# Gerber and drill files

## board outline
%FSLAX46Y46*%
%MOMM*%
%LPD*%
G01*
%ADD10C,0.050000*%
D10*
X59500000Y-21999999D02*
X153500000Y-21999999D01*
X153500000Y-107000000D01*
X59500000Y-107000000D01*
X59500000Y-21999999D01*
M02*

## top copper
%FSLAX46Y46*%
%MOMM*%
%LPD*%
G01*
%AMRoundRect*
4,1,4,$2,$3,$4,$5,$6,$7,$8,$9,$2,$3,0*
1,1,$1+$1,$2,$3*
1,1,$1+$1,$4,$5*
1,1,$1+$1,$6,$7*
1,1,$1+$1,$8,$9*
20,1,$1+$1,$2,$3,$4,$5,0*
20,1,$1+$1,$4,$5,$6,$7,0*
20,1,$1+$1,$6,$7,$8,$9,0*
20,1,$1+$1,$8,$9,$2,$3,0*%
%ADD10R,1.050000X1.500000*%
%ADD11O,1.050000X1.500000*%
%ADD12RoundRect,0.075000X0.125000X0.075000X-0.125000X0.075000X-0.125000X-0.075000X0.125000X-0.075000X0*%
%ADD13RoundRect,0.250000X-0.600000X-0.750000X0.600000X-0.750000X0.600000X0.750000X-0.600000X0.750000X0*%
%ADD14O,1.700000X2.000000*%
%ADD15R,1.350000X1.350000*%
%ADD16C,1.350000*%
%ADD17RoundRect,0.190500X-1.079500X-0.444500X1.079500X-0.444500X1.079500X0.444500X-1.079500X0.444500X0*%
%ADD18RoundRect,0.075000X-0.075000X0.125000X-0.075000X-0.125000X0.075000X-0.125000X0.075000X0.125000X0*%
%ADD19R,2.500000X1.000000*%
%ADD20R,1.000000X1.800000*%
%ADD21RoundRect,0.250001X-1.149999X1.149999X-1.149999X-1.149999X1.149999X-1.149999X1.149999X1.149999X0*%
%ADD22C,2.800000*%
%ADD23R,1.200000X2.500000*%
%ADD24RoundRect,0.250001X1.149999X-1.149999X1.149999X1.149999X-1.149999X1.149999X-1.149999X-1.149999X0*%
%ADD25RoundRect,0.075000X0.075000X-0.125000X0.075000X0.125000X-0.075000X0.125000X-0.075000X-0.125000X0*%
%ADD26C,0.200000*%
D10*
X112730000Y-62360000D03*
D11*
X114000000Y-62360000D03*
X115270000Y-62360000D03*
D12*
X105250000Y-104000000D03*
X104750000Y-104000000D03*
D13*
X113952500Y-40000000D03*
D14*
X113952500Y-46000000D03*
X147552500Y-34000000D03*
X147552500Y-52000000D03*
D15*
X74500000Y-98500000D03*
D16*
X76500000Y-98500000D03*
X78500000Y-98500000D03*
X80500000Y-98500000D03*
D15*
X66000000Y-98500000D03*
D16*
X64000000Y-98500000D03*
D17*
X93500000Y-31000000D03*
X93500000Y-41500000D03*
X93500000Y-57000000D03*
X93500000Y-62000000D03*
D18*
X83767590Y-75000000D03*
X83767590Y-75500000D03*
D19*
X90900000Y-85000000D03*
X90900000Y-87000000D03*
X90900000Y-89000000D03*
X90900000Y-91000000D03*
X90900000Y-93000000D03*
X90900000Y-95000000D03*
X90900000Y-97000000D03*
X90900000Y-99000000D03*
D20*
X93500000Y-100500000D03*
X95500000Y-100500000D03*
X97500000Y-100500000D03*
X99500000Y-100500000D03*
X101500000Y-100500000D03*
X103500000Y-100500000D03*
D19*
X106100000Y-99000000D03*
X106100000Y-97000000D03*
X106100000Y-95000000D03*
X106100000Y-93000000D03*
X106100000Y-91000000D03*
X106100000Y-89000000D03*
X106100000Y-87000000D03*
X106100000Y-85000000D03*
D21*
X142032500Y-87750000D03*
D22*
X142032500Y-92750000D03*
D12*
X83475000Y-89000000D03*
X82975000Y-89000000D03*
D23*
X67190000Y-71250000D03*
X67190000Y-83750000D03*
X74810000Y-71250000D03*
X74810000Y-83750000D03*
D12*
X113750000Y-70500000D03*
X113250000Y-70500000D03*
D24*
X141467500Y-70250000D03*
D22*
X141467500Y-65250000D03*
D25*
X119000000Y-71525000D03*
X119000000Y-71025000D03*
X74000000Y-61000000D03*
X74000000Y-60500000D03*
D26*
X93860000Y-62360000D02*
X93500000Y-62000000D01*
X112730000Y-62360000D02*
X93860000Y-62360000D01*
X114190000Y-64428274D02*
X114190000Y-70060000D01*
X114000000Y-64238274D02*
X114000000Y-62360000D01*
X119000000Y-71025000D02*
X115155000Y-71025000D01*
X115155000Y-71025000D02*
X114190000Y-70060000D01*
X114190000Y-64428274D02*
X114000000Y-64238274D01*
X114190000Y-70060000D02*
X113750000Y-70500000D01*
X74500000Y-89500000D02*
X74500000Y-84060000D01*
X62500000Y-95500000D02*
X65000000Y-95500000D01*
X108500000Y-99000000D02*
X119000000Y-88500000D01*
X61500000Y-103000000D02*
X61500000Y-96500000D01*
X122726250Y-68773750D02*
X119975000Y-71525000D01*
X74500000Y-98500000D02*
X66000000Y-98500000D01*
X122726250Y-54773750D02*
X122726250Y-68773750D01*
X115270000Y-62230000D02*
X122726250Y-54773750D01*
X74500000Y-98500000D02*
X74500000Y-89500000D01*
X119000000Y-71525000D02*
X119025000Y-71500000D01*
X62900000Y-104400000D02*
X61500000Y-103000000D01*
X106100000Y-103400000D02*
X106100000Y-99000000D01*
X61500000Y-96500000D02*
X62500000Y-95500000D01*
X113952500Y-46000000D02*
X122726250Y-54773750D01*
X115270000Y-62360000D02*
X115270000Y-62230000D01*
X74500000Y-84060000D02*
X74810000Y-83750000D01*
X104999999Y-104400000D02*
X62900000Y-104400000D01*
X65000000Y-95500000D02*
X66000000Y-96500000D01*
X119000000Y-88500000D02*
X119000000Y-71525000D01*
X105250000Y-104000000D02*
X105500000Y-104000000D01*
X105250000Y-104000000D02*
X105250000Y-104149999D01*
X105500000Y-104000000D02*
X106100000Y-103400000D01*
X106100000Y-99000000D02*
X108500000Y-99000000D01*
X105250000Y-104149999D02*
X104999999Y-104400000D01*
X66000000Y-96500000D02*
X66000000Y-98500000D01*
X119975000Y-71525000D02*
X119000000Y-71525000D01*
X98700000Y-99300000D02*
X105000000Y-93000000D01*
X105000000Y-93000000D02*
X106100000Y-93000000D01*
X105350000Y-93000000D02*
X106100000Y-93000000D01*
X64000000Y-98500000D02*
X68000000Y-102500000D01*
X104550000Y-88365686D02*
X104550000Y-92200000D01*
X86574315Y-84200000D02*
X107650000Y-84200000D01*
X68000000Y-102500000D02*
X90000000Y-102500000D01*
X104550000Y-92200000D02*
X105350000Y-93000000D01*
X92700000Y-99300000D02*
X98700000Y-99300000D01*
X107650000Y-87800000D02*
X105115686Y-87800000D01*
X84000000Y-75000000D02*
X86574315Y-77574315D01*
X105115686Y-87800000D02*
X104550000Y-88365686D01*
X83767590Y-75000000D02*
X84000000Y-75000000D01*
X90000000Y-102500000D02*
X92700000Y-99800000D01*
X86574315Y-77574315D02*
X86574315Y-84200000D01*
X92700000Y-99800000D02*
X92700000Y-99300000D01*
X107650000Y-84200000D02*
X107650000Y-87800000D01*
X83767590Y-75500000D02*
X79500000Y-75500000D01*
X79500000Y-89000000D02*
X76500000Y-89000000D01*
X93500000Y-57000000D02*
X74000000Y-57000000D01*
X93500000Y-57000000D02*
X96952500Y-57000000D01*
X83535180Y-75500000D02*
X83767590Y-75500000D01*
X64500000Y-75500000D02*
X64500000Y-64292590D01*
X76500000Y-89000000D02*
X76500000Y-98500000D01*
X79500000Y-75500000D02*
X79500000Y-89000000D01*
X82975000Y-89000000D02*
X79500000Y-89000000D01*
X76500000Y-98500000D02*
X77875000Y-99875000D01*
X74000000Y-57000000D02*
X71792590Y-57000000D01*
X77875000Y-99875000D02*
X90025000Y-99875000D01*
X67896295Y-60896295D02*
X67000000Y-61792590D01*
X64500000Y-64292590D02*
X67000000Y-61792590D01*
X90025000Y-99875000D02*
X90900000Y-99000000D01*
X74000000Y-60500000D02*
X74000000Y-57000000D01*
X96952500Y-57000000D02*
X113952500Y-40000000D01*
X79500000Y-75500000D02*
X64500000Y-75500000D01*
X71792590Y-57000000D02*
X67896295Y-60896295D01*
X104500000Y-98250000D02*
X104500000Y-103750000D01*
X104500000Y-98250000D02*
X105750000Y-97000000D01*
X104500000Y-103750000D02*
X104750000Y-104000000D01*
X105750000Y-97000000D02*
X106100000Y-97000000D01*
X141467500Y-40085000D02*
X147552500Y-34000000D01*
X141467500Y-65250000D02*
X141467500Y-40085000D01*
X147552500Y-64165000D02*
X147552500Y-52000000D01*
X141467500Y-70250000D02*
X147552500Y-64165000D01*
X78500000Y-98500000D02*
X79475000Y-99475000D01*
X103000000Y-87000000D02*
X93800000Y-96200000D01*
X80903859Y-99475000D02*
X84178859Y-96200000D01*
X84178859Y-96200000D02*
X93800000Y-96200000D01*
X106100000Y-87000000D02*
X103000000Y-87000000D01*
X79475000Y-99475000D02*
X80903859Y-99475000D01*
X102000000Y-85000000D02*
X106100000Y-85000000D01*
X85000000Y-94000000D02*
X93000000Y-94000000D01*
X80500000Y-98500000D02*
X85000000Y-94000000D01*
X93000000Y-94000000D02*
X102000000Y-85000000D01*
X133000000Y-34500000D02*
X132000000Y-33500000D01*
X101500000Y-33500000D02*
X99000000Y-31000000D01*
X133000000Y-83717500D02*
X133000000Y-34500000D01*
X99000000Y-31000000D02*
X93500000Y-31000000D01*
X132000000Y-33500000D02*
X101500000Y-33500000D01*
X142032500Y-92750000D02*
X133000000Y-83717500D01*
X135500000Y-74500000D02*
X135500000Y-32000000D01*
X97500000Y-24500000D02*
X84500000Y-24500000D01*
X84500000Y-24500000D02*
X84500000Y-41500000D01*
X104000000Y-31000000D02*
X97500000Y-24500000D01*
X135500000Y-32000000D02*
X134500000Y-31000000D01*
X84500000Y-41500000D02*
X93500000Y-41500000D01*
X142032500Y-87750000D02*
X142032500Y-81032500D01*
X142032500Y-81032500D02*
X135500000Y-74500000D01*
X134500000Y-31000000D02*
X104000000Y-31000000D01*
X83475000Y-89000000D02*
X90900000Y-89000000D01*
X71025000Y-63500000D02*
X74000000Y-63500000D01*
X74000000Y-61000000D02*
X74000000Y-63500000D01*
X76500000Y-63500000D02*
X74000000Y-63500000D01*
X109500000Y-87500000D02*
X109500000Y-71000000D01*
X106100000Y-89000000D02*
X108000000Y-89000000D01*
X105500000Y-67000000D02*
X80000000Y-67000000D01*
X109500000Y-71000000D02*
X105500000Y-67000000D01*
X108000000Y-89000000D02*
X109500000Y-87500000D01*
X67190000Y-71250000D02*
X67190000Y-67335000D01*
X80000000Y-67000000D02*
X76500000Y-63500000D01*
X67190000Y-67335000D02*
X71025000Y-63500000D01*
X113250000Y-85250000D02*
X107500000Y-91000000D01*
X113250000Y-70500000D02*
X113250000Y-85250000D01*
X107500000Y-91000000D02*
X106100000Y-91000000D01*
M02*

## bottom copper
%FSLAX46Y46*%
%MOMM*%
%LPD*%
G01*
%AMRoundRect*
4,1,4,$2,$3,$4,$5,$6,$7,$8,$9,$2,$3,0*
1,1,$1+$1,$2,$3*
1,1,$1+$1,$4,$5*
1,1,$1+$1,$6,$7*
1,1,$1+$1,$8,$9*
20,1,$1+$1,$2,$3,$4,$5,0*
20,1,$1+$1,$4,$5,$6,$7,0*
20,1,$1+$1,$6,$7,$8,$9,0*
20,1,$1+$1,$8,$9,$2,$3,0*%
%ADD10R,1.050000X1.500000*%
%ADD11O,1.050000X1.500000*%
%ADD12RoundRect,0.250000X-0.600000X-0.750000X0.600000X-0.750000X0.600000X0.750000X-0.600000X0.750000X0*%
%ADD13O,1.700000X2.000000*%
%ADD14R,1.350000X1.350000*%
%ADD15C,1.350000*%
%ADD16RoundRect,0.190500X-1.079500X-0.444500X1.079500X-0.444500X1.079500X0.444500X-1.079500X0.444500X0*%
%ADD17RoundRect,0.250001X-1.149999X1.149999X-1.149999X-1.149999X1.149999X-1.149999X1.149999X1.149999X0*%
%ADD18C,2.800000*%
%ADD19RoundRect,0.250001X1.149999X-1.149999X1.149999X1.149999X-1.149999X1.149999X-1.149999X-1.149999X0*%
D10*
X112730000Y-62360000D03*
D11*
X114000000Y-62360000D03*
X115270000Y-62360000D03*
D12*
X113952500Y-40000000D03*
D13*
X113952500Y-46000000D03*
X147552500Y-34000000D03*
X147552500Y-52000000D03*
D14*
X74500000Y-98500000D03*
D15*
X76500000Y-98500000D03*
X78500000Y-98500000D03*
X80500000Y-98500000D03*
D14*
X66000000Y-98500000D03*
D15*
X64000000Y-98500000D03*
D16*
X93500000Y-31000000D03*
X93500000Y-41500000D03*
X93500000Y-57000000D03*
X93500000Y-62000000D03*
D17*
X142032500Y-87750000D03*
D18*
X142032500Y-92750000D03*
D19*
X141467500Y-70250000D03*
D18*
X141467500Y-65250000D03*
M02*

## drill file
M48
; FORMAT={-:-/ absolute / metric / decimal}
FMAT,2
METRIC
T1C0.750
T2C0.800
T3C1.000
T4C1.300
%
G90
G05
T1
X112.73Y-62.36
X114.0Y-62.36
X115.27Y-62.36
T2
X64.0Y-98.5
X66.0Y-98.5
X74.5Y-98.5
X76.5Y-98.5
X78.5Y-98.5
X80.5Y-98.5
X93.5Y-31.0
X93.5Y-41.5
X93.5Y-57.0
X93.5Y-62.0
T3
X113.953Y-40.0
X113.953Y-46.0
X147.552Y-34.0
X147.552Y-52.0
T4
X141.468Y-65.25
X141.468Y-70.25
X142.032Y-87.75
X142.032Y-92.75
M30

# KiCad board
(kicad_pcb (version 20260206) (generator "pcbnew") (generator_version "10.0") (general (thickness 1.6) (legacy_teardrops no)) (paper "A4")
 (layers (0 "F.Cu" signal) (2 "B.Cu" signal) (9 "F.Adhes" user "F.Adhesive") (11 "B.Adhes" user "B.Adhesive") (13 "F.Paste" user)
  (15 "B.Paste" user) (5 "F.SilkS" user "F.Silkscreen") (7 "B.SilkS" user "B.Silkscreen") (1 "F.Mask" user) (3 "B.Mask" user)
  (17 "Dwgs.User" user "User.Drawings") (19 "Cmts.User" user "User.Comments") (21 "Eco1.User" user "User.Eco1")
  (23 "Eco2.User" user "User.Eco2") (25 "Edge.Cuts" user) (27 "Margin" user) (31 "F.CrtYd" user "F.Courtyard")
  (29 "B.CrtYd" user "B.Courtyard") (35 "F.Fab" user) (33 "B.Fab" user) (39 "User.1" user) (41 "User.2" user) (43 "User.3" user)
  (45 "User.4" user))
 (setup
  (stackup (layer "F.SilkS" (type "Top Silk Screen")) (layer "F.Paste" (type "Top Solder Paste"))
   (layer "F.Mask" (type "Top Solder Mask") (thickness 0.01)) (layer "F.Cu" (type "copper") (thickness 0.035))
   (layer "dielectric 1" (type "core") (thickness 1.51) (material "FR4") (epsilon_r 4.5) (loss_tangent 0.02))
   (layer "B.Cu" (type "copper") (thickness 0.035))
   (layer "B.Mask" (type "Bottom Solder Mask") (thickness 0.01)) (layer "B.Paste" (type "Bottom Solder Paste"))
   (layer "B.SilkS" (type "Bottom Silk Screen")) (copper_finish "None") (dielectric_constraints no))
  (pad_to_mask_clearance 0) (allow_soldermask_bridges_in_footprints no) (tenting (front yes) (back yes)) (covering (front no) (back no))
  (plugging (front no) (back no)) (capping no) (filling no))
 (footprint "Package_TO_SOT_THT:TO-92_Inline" (layer "F.Cu") (at 112.73 62.36)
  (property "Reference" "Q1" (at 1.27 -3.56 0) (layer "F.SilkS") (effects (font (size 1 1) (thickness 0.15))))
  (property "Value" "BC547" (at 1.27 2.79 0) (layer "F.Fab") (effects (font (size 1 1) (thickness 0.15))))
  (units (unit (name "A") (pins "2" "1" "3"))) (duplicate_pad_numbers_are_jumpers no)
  (pad "1" thru_hole rect (at 0 0) (size 1.05 1.5) (drill 0.75) (layers "*.Cu" "*.Mask") (remove_unused_layers no) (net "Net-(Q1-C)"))
  (pad "2" thru_hole oval (at 1.27 0) (size 1.05 1.5) (drill 0.75) (layers "*.Cu" "*.Mask") (remove_unused_layers no) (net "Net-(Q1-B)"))
  (pad "3" thru_hole oval (at 2.54 0) (size 1.05 1.5) (drill 0.75) (layers "*.Cu" "*.Mask") (remove_unused_layers no) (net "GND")))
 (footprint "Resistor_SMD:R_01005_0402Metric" (layer "F.Cu") (at 105 104 180)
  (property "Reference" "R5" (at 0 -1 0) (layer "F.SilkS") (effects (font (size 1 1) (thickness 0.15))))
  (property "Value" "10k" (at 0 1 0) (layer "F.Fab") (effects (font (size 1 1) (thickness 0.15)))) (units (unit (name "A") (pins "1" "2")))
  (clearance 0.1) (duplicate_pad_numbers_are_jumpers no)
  (pad "" smd roundrect (at -0.275 0 180) (size 0.27 0.27) (layers "F.Paste") (roundrect_rratio 0.25))
  (pad "" smd roundrect (at 0.275 0 180) (size 0.27 0.27) (layers "F.Paste") (roundrect_rratio 0.25))
  (pad "1" smd roundrect (at -0.25 0 180) (size 0.4 0.3) (layers "F.Cu" "F.Mask") (roundrect_rratio 0.25) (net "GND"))
  (pad "2" smd roundrect (at 0.25 0 180) (size 0.4 0.3) (layers "F.Cu" "F.Mask") (roundrect_rratio 0.25) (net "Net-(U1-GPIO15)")))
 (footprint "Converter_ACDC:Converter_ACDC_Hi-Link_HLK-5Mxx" (layer "F.Cu") (at 113.9525 40)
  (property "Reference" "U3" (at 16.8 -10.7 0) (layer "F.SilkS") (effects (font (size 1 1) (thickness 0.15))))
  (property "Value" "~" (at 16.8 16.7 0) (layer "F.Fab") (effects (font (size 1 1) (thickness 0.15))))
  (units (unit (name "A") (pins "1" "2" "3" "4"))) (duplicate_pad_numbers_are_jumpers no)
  (pad "1" thru_hole roundrect (at 0 0) (size 1.7 2) (drill 1) (layers "*.Cu" "*.Mask") (remove_unused_layers no)
   (roundrect_rratio 0.147059) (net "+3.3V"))
  (pad "2" thru_hole oval (at 0 6) (size 1.7 2) (drill 1) (layers "*.Cu" "*.Mask") (remove_unused_layers no) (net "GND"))
  (pad "3" thru_hole oval (at 33.6 -6) (size 1.7 2) (drill 1) (layers "*.Cu" "*.Mask") (remove_unused_layers no) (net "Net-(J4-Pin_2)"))
  (pad "4" thru_hole oval (at 33.6 12) (size 1.7 2) (drill 1) (layers "*.Cu" "*.Mask") (remove_unused_layers no) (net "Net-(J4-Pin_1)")))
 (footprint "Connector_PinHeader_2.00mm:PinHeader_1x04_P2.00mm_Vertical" (layer "F.Cu") (at 74.5 98.5 90)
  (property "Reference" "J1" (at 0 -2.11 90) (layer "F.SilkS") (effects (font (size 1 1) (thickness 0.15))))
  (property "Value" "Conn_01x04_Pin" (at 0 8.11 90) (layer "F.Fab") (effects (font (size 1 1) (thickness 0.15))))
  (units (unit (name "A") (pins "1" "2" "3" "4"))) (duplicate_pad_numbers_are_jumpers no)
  (pad "1" thru_hole rect (at 0 0 90) (size 1.35 1.35) (drill 0.8) (layers "*.Cu" "*.Mask") (remove_unused_layers no) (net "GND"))
  (pad "2" thru_hole circle (at 0 2 90) (size 1.35 1.35) (drill 0.8) (layers "*.Cu" "*.Mask") (remove_unused_layers no) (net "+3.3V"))
  (pad "3" thru_hole circle (at 0 4 90) (size 1.35 1.35) (drill 0.8) (layers "*.Cu" "*.Mask") (remove_unused_layers no)
   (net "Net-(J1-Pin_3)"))
  (pad "4" thru_hole circle (at 0 6 90) (size 1.35 1.35) (drill 0.8) (layers "*.Cu" "*.Mask") (remove_unused_layers no)
   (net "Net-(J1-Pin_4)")))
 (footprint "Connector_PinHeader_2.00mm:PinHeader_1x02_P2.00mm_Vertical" (layer "F.Cu") (at 66 98.5 -90)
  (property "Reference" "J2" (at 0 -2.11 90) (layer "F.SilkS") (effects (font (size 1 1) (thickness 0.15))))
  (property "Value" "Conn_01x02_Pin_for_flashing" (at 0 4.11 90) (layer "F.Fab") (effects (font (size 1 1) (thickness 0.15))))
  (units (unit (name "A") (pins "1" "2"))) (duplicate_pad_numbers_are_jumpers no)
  (pad "1" thru_hole rect (at 0 0 270) (size 1.35 1.35) (drill 0.8) (layers "*.Cu" "*.Mask") (remove_unused_layers no) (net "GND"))
  (pad "2" thru_hole circle (at 0 2 270) (size 1.35 1.35) (drill 0.8) (layers "*.Cu" "*.Mask") (remove_unused_layers no)
   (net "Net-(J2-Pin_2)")))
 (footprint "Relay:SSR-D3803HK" (layer "F.Cu") (at 93.5 46.5)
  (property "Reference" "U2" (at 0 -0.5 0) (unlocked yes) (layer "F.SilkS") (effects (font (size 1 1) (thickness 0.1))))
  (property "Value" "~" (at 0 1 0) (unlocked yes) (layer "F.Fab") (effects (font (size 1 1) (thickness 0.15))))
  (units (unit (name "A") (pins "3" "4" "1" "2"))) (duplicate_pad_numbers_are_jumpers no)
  (pad "1" thru_hole roundrect (at 0 -15.5) (size 2.54 1.27) (drill 0.8) (layers "*.Cu" "*.Mask") (remove_unused_layers no)
   (roundrect_rratio 0.15) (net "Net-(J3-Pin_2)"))
  (pad "2" thru_hole roundrect (at 0 -5) (size 2.54 1.27) (drill 0.8) (layers "*.Cu" "*.Mask") (remove_unused_layers no)
   (roundrect_rratio 0.15) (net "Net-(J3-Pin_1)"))
  (pad "3" thru_hole roundrect (at 0 10.5) (size 2.54 1.27) (drill 0.8) (layers "*.Cu" "*.Mask") (remove_unused_layers no)
   (roundrect_rratio 0.15) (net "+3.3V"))
  (pad "4" thru_hole roundrect (at 0 15.5) (size 2.54 1.27) (drill 0.8) (layers "*.Cu" "*.Mask") (remove_unused_layers no)
   (roundrect_rratio 0.15) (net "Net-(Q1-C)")))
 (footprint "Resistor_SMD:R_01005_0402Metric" (layer "F.Cu") (at 83.76759 75.25 -90)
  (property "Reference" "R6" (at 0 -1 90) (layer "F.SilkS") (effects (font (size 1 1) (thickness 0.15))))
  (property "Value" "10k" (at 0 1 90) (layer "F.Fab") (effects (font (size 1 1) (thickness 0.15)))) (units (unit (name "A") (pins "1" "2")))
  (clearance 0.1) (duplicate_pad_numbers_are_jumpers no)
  (pad "" smd roundrect (at -0.275 0 270) (size 0.27 0.27) (layers "F.Paste") (roundrect_rratio 0.25))
  (pad "" smd roundrect (at 0.275 0 270) (size 0.27 0.27) (layers "F.Paste") (roundrect_rratio 0.25))
  (pad "1" smd roundrect (at -0.25 0 270) (size 0.4 0.3) (layers "F.Cu" "F.Mask") (roundrect_rratio 0.25) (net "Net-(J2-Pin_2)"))
  (pad "2" smd roundrect (at 0.25 0 270) (size 0.4 0.3) (layers "F.Cu" "F.Mask") (roundrect_rratio 0.25) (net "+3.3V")))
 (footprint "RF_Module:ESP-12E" (layer "F.Cu") (at 98.5 88.5)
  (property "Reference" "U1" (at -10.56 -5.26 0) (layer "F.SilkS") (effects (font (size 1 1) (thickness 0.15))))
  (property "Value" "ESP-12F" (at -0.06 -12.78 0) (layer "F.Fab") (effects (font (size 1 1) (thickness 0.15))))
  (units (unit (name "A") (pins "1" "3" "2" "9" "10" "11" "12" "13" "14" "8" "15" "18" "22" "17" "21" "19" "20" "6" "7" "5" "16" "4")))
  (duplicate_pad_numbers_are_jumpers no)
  (pad "1" smd rect (at -7.6 -3.5) (size 2.5 1) (layers "F.Cu" "F.Mask" "F.Paste") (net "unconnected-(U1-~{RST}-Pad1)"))
  (pad "2" smd rect (at -7.6 -1.5) (size 2.5 1) (layers "F.Cu" "F.Mask" "F.Paste") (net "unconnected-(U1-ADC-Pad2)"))
  (pad "3" smd rect (at -7.6 0.5) (size 2.5 1) (layers "F.Cu" "F.Mask" "F.Paste") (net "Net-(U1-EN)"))
  (pad "4" smd rect (at -7.6 2.5) (size 2.5 1) (layers "F.Cu" "F.Mask" "F.Paste") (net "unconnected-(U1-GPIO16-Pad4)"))
  (pad "5" smd rect (at -7.6 4.5) (size 2.5 1) (layers "F.Cu" "F.Mask" "F.Paste") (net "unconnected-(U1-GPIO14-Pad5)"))
  (pad "6" smd rect (at -7.6 6.5) (size 2.5 1) (layers "F.Cu" "F.Mask" "F.Paste") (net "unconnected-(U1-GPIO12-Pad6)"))
  (pad "7" smd rect (at -7.6 8.5) (size 2.5 1) (layers "F.Cu" "F.Mask" "F.Paste") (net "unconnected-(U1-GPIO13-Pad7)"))
  (pad "8" smd rect (at -7.6 10.5) (size 2.5 1) (layers "F.Cu" "F.Mask" "F.Paste") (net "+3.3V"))
  (pad "9" smd rect (at -5 12) (size 1 1.8) (layers "F.Cu" "F.Mask" "F.Paste") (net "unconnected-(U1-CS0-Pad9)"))
  (pad "10" smd rect (at -3 12) (size 1 1.8) (layers "F.Cu" "F.Mask" "F.Paste") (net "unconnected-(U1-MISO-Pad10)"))
  (pad "11" smd rect (at -1 12) (size 1 1.8) (layers "F.Cu" "F.Mask" "F.Paste") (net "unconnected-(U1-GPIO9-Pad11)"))
  (pad "12" smd rect (at 1 12) (size 1 1.8) (layers "F.Cu" "F.Mask" "F.Paste") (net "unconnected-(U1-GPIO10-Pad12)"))
  (pad "13" smd rect (at 3 12) (size 1 1.8) (layers "F.Cu" "F.Mask" "F.Paste") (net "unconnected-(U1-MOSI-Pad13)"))
  (pad "14" smd rect (at 5 12) (size 1 1.8) (layers "F.Cu" "F.Mask" "F.Paste") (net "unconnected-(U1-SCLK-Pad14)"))
  (pad "15" smd rect (at 7.6 10.5) (size 2.5 1) (layers "F.Cu" "F.Mask" "F.Paste") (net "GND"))
  (pad "16" smd rect (at 7.6 8.5) (size 2.5 1) (layers "F.Cu" "F.Mask" "F.Paste") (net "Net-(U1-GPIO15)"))
  (pad "17" smd rect (at 7.6 6.5) (size 2.5 1) (layers "F.Cu" "F.Mask" "F.Paste") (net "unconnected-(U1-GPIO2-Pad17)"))
  (pad "18" smd rect (at 7.6 4.5) (size 2.5 1) (layers "F.Cu" "F.Mask" "F.Paste") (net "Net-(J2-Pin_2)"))
  (pad "19" smd rect (at 7.6 2.5) (size 2.5 1) (layers "F.Cu" "F.Mask" "F.Paste") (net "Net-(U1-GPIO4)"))
  (pad "20" smd rect (at 7.6 0.5) (size 2.5 1) (layers "F.Cu" "F.Mask" "F.Paste") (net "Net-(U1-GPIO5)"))
  (pad "21" smd rect (at 7.6 -1.5) (size 2.5 1) (layers "F.Cu" "F.Mask" "F.Paste") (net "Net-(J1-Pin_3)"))
  (pad "22" smd rect (at 7.6 -3.5) (size 2.5 1) (layers "F.Cu" "F.Mask" "F.Paste") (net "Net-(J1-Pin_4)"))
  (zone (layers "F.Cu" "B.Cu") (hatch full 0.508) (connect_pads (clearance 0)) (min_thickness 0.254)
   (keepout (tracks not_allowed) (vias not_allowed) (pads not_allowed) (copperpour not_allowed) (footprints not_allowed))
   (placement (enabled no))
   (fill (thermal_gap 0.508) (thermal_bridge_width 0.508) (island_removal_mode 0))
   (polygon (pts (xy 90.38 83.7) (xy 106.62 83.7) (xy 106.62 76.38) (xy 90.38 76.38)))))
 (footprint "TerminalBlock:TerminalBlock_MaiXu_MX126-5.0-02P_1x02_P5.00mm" (layer "F.Cu") (at 142.0325 87.75 -90)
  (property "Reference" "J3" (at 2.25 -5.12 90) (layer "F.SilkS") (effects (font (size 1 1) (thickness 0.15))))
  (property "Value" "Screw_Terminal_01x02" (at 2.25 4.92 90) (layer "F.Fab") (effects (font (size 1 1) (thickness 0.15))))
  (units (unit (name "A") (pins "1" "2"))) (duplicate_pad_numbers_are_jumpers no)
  (pad "1" thru_hole roundrect (at 0 0 270) (size 2.8 2.8) (drill 1.3) (layers "*.Cu" "*.Mask") (remove_unused_layers no)
   (roundrect_rratio 0.089286) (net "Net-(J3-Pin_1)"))
  (pad "2" thru_hole circle (at 5 0 270) (size 2.8 2.8) (drill 1.3) (layers "*.Cu" "*.Mask") (remove_unused_layers no)
   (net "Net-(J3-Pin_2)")))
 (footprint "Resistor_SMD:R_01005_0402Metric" (layer "F.Cu") (at 83.225 89 180)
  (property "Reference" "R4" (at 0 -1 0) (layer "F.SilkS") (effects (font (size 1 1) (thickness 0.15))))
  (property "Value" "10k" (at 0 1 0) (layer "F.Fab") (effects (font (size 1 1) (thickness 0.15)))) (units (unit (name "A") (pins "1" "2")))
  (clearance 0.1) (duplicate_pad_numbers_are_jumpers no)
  (pad "" smd roundrect (at -0.275 0 180) (size 0.27 0.27) (layers "F.Paste") (roundrect_rratio 0.25))
  (pad "" smd roundrect (at 0.275 0 180) (size 0.27 0.27) (layers "F.Paste") (roundrect_rratio 0.25))
  (pad "1" smd roundrect (at -0.25 0 180) (size 0.4 0.3) (layers "F.Cu" "F.Mask") (roundrect_rratio 0.25) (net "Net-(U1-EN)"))
  (pad "2" smd roundrect (at 0.25 0 180) (size 0.4 0.3) (layers "F.Cu" "F.Mask") (roundrect_rratio 0.25) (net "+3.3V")))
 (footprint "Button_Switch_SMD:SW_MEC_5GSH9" (layer "F.Cu") (at 71 77.5)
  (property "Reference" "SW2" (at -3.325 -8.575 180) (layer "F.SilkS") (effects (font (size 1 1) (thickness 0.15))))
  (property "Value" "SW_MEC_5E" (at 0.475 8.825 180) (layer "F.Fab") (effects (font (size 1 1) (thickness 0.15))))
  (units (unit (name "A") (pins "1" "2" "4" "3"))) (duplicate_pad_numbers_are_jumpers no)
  (pad "1" smd rect (at -3.81 -6.25 90) (size 2.5 1.2) (layers "F.Cu" "F.Mask" "F.Paste") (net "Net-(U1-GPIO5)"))
  (pad "2" smd rect (at -3.81 6.25 90) (size 2.5 1.2) (layers "F.Cu" "F.Mask" "F.Paste") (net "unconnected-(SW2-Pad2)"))
  (pad "3" smd rect (at 3.81 -6.25 90) (size 2.5 1.2) (layers "F.Cu" "F.Mask" "F.Paste") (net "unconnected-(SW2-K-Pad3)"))
  (pad "4" smd rect (at 3.81 6.25 90) (size 2.5 1.2) (layers "F.Cu" "F.Mask" "F.Paste") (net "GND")))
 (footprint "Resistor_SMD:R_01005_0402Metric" (layer "F.Cu") (at 113.5 70.5 180)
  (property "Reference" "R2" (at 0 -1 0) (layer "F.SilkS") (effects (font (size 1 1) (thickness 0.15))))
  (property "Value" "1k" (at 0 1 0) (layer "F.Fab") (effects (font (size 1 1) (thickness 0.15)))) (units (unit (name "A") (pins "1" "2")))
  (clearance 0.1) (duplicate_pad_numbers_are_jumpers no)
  (pad "" smd roundrect (at -0.275 0 180) (size 0.27 0.27) (layers "F.Paste") (roundrect_rratio 0.25))
  (pad "" smd roundrect (at 0.275 0 180) (size 0.27 0.27) (layers "F.Paste") (roundrect_rratio 0.25))
  (pad "1" smd roundrect (at -0.25 0 180) (size 0.4 0.3) (layers "F.Cu" "F.Mask") (roundrect_rratio 0.25) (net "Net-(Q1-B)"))
  (pad "2" smd roundrect (at 0.25 0 180) (size 0.4 0.3) (layers "F.Cu" "F.Mask") (roundrect_rratio 0.25) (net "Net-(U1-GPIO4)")))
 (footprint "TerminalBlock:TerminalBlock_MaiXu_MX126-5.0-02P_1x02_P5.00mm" (layer "F.Cu") (at 141.4675 70.25 90)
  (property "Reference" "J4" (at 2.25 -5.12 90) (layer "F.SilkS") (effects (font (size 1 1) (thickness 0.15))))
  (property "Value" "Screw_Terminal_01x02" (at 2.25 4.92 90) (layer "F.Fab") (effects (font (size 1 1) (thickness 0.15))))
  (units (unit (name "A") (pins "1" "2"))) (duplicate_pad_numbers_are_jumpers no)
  (pad "1" thru_hole roundrect (at 0 0 90) (size 2.8 2.8) (drill 1.3) (layers "*.Cu" "*.Mask") (remove_unused_layers no)
   (roundrect_rratio 0.089286) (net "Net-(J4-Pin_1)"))
  (pad "2" thru_hole circle (at 5 0 90) (size 2.8 2.8) (drill 1.3) (layers "*.Cu" "*.Mask") (remove_unused_layers no) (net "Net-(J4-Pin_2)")))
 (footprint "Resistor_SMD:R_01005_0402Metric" (layer "F.Cu") (at 119 71.275 90)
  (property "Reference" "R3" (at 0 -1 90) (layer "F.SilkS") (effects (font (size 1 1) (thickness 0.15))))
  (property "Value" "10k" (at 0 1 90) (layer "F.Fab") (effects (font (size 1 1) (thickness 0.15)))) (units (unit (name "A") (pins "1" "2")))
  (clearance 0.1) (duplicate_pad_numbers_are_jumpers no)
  (pad "" smd roundrect (at -0.275 0 90) (size 0.27 0.27) (layers "F.Paste") (roundrect_rratio 0.25))
  (pad "" smd roundrect (at 0.275 0 90) (size 0.27 0.27) (layers "F.Paste") (roundrect_rratio 0.25))
  (pad "1" smd roundrect (at -0.25 0 90) (size 0.4 0.3) (layers "F.Cu" "F.Mask") (roundrect_rratio 0.25) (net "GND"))
  (pad "2" smd roundrect (at 0.25 0 90) (size 0.4 0.3) (layers "F.Cu" "F.Mask") (roundrect_rratio 0.25) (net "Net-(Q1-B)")))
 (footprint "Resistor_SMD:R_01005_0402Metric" (layer "F.Cu") (at 74 60.75 90)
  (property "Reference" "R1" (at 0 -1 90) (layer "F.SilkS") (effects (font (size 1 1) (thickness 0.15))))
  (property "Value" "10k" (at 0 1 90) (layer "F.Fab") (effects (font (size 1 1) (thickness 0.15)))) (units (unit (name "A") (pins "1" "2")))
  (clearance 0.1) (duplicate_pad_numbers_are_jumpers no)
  (pad "" smd roundrect (at -0.275 0 90) (size 0.27 0.27) (layers "F.Paste") (roundrect_rratio 0.25))
  (pad "" smd roundrect (at 0.275 0 90) (size 0.27 0.27) (layers "F.Paste") (roundrect_rratio 0.25))
  (pad "1" smd roundrect (at -0.25 0 90) (size 0.4 0.3) (layers "F.Cu" "F.Mask") (roundrect_rratio 0.25) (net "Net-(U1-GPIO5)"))
  (pad "2" smd roundrect (at 0.25 0 90) (size 0.4 0.3) (layers "F.Cu" "F.Mask") (roundrect_rratio 0.25) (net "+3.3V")))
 (gr_rect (start 59.5 21.999999) (end 153.5 107) (stroke (width 0.05) (type default)) (fill no) (layer "Edge.Cuts"))
 (segment (start 93.86 62.36) (end 93.5 62) (width 0.2) (layer "F.Cu") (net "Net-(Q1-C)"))
 (segment (start 112.73 62.36) (end 93.86 62.36) (width 0.2) (layer "F.Cu") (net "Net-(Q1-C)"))
 (segment (start 114.19 64.428274) (end 114.19 70.06) (width 0.2) (layer "F.Cu") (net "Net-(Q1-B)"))
 (segment (start 114 64.238274) (end 114 62.36) (width 0.2) (layer "F.Cu") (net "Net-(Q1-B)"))
 (segment (start 119 71.025) (end 115.155 71.025) (width 0.2) (layer "F.Cu") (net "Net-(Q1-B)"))
 (segment (start 115.155 71.025) (end 114.19 70.06) (width 0.2) (layer "F.Cu") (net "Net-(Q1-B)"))
 (segment (start 114.19 64.428274) (end 114 64.238274) (width 0.2) (layer "F.Cu") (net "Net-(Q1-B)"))
 (segment (start 114.19 70.06) (end 113.75 70.5) (width 0.2) (layer "F.Cu") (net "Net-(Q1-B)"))
 (segment (start 74.5 89.5) (end 74.5 84.06) (width 0.2) (layer "F.Cu") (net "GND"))
 (segment (start 62.5 95.5) (end 65 95.5) (width 0.2) (layer "F.Cu") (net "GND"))
 (segment (start 108.5 99) (end 119 88.5) (width 0.2) (layer "F.Cu") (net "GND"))
 (segment (start 61.5 103) (end 61.5 96.5) (width 0.2) (layer "F.Cu") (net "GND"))
 (segment (start 122.72625 68.77375) (end 119.975 71.525) (width 0.2) (layer "F.Cu") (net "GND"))
 (segment (start 74.5 98.5) (end 66 98.5) (width 0.2) (layer "F.Cu") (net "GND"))
 (segment (start 122.72625 54.77375) (end 122.72625 68.77375) (width 0.2) (layer "F.Cu") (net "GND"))
 (segment (start 115.27 62.23) (end 122.72625 54.77375) (width 0.2) (layer "F.Cu") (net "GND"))
 (segment (start 74.5 98.5) (end 74.5 89.5) (width 0.2) (layer "F.Cu") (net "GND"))
 (segment (start 119 71.525) (end 119.025 71.5) (width 0.2) (layer "F.Cu") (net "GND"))
 (segment (start 62.9 104.4) (end 61.5 103) (width 0.2) (layer "F.Cu") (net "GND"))
 (segment (start 106.1 103.4) (end 106.1 99) (width 0.2) (layer "F.Cu") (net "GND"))
 (segment (start 61.5 96.5) (end 62.5 95.5) (width 0.2) (layer "F.Cu") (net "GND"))
 (segment (start 113.9525 46) (end 122.72625 54.77375) (width 0.2) (layer "F.Cu") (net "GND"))
 (segment (start 115.27 62.36) (end 115.27 62.23) (width 0.2) (layer "F.Cu") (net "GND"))
 (segment (start 74.5 84.06) (end 74.81 83.75) (width 0.2) (layer "F.Cu") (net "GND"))
 (segment (start 104.999999 104.4) (end 62.9 104.4) (width 0.2) (layer "F.Cu") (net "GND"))
 (segment (start 65 95.5) (end 66 96.5) (width 0.2) (layer "F.Cu") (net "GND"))
 (segment (start 119 88.5) (end 119 71.525) (width 0.2) (layer "F.Cu") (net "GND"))
 (segment (start 105.25 104) (end 105.5 104) (width 0.2) (layer "F.Cu") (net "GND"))
 (segment (start 105.25 104) (end 105.25 104.149999) (width 0.2) (layer "F.Cu") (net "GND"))
 (segment (start 105.5 104) (end 106.1 103.4) (width 0.2) (layer "F.Cu") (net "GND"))
 (segment (start 106.1 99) (end 108.5 99) (width 0.2) (layer "F.Cu") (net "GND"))
 (segment (start 105.25 104.149999) (end 104.999999 104.4) (width 0.2) (layer "F.Cu") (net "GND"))
 (segment (start 66 96.5) (end 66 98.5) (width 0.2) (layer "F.Cu") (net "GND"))
 (segment (start 119.975 71.525) (end 119 71.525) (width 0.2) (layer "F.Cu") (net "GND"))
 (segment (start 98.7 99.3) (end 105 93) (width 0.2) (layer "F.Cu") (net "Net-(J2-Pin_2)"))
 (segment (start 105 93) (end 106.1 93) (width 0.2) (layer "F.Cu") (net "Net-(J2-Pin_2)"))
 (segment (start 105.35 93) (end 106.1 93) (width 0.2) (layer "F.Cu") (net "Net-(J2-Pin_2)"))
 (segment (start 64 98.5) (end 68 102.5) (width 0.2) (layer "F.Cu") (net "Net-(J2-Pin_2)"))
 (segment (start 104.55 88.365686) (end 104.55 92.2) (width 0.2) (layer "F.Cu") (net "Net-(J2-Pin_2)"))
 (segment (start 86.574315 84.2) (end 107.65 84.2) (width 0.2) (layer "F.Cu") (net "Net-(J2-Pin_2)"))
 (segment (start 68 102.5) (end 90 102.5) (width 0.2) (layer "F.Cu") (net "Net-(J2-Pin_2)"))
 (segment (start 104.55 92.2) (end 105.35 93) (width 0.2) (layer "F.Cu") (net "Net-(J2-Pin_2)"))
 (segment (start 92.7 99.3) (end 98.7 99.3) (width 0.2) (layer "F.Cu") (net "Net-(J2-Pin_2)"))
 (segment (start 107.65 87.8) (end 105.115686 87.8) (width 0.2) (layer "F.Cu") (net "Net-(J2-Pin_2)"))
 (segment (start 84 75) (end 86.574315 77.574315) (width 0.2) (layer "F.Cu") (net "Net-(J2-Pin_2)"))
 (segment (start 105.115686 87.8) (end 104.55 88.365686) (width 0.2) (layer "F.Cu") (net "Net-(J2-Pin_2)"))
 (segment (start 83.76759 75) (end 84 75) (width 0.2) (layer "F.Cu") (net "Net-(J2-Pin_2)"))
 (segment (start 90 102.5) (end 92.7 99.8) (width 0.2) (layer "F.Cu") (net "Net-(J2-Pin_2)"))
 (segment (start 86.574315 77.574315) (end 86.574315 84.2) (width 0.2) (layer "F.Cu") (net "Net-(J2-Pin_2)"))
 (segment (start 92.7 99.8) (end 92.7 99.3) (width 0.2) (layer "F.Cu") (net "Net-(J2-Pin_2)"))
 (segment (start 107.65 84.2) (end 107.65 87.8) (width 0.2) (layer "F.Cu") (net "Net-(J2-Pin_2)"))
 (segment (start 83.76759 75.5) (end 79.5 75.5) (width 0.2) (layer "F.Cu") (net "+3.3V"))
 (segment (start 79.5 89) (end 76.5 89) (width 0.2) (layer "F.Cu") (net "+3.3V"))
 (segment (start 93.5 57) (end 74 57) (width 0.2) (layer "F.Cu") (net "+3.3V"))
 (segment (start 93.5 57) (end 96.9525 57) (width 0.2) (layer "F.Cu") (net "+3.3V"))
 (segment (start 83.53518 75.5) (end 83.76759 75.5) (width 0.2) (layer "F.Cu") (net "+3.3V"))
 (segment (start 64.5 75.5) (end 64.5 64.29259) (width 0.2) (layer "F.Cu") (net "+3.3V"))
 (segment (start 76.5 89) (end 76.5 98.5) (width 0.2) (layer "F.Cu") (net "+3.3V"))
 (segment (start 79.5 75.5) (end 79.5 89) (width 0.2) (layer "F.Cu") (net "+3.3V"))
 (segment (start 82.975 89) (end 79.5 89) (width 0.2) (layer "F.Cu") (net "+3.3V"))
 (segment (start 76.5 98.5) (end 77.875 99.875) (width 0.2) (layer "F.Cu") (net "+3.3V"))
 (segment (start 74 57) (end 71.79259 57) (width 0.2) (layer "F.Cu") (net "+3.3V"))
 (segment (start 77.875 99.875) (end 90.025 99.875) (width 0.2) (layer "F.Cu") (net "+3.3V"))
 (segment (start 67.896295 60.896295) (end 67 61.79259) (width 0.2) (layer "F.Cu") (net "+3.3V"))
 (segment (start 64.5 64.29259) (end 67 61.79259) (width 0.2) (layer "F.Cu") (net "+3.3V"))
 (segment (start 90.025 99.875) (end 90.9 99) (width 0.2) (layer "F.Cu") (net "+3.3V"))
 (segment (start 74 60.5) (end 74 57) (width 0.2) (layer "F.Cu") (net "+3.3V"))
 (segment (start 96.9525 57) (end 113.9525 40) (width 0.2) (layer "F.Cu") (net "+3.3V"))
 (segment (start 79.5 75.5) (end 64.5 75.5) (width 0.2) (layer "F.Cu") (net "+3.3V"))
 (segment (start 71.79259 57) (end 67.896295 60.896295) (width 0.2) (layer "F.Cu") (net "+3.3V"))
 (segment (start 104.5 98.25) (end 104.5 103.75) (width 0.2) (layer "F.Cu") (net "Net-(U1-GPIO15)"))
 (segment (start 104.5 98.25) (end 105.75 97) (width 0.2) (layer "F.Cu") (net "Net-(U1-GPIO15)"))
 (segment (start 104.5 103.75) (end 104.75 104) (width 0.2) (layer "F.Cu") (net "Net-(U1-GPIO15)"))
 (segment (start 105.75 97) (end 106.1 97) (width 0.2) (layer "F.Cu") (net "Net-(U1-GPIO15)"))
 (segment (start 141.4675 40.085) (end 147.5525 34) (width 0.2) (layer "F.Cu") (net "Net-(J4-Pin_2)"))
 (segment (start 141.4675 65.25) (end 141.4675 40.085) (width 0.2) (layer "F.Cu") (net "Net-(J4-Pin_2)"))
 (segment (start 147.5525 64.165) (end 147.5525 52) (width 0.2) (layer "F.Cu") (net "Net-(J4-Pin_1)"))
 (segment (start 141.4675 70.25) (end 147.5525 64.165) (width 0.2) (layer "F.Cu") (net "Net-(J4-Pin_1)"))
 (segment (start 78.5 98.5) (end 79.475 99.475) (width 0.2) (layer "F.Cu") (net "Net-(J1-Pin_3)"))
 (segment (start 103 87) (end 93.8 96.2) (width 0.2) (layer "F.Cu") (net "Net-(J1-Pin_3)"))
 (segment (start 80.903859 99.475) (end 84.178859 96.2) (width 0.2) (layer "F.Cu") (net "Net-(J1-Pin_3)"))
 (segment (start 84.178859 96.2) (end 93.8 96.2) (width 0.2) (layer "F.Cu") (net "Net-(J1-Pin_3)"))
 (segment (start 106.1 87) (end 103 87) (width 0.2) (layer "F.Cu") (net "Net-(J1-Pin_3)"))
 (segment (start 79.475 99.475) (end 80.903859 99.475) (width 0.2) (layer "F.Cu") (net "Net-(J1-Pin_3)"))
 (segment (start 102 85) (end 106.1 85) (width 0.2) (layer "F.Cu") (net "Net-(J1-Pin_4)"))
 (segment (start 85 94) (end 93 94) (width 0.2) (layer "F.Cu") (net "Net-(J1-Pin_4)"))
 (segment (start 80.5 98.5) (end 85 94) (width 0.2) (layer "F.Cu") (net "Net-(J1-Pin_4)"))
 (segment (start 93 94) (end 102 85) (width 0.2) (layer "F.Cu") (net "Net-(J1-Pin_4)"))
 (segment (start 133 34.5) (end 132 33.5) (width 0.2) (layer "F.Cu") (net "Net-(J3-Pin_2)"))
 (segment (start 101.5 33.5) (end 99 31) (width 0.2) (layer "F.Cu") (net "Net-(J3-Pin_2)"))
 (segment (start 133 83.7175) (end 133 34.5) (width 0.2) (layer "F.Cu") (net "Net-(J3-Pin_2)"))
 (segment (start 99 31) (end 93.5 31) (width 0.2) (layer "F.Cu") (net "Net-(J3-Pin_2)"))
 (segment (start 132 33.5) (end 101.5 33.5) (width 0.2) (layer "F.Cu") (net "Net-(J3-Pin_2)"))
 (segment (start 142.0325 92.75) (end 133 83.7175) (width 0.2) (layer "F.Cu") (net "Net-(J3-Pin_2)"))
 (segment (start 135.5 74.5) (end 135.5 32) (width 0.2) (layer "F.Cu") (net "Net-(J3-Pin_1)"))
 (segment (start 97.5 24.5) (end 84.5 24.5) (width 0.2) (layer "F.Cu") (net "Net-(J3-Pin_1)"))
 (segment (start 84.5 24.5) (end 84.5 41.5) (width 0.2) (layer "F.Cu") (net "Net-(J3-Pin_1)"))
 (segment (start 104 31) (end 97.5 24.5) (width 0.2) (layer "F.Cu") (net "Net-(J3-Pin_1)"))
 (segment (start 135.5 32) (end 134.5 31) (width 0.2) (layer "F.Cu") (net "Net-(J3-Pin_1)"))
 (segment (start 84.5 41.5) (end 93.5 41.5) (width 0.2) (layer "F.Cu") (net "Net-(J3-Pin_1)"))
 (segment (start 142.0325 87.75) (end 142.0325 81.0325) (width 0.2) (layer "F.Cu") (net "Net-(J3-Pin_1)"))
 (segment (start 142.0325 81.0325) (end 135.5 74.5) (width 0.2) (layer "F.Cu") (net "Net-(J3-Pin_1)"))
 (segment (start 134.5 31) (end 104 31) (width 0.2) (layer "F.Cu") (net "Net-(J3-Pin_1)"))
 (segment (start 83.475 89) (end 90.9 89) (width 0.2) (layer "F.Cu") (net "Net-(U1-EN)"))
 (segment (start 71.025 63.5) (end 74 63.5) (width 0.2) (layer "F.Cu") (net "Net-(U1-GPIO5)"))
 (segment (start 74 61) (end 74 63.5) (width 0.2) (layer "F.Cu") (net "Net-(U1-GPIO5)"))
 (segment (start 76.5 63.5) (end 74 63.5) (width 0.2) (layer "F.Cu") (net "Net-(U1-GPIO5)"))
 (segment (start 109.5 87.5) (end 109.5 71) (width 0.2) (layer "F.Cu") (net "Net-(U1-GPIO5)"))
 (segment (start 106.1 89) (end 108 89) (width 0.2) (layer "F.Cu") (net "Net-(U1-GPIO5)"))
 (segment (start 105.5 67) (end 80 67) (width 0.2) (layer "F.Cu") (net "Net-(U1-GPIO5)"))
 (segment (start 109.5 71) (end 105.5 67) (width 0.2) (layer "F.Cu") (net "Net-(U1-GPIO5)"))
 (segment (start 108 89) (end 109.5 87.5) (width 0.2) (layer "F.Cu") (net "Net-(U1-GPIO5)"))
 (segment (start 67.19 71.25) (end 67.19 67.335) (width 0.2) (layer "F.Cu") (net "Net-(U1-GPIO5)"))
 (segment (start 80 67) (end 76.5 63.5) (width 0.2) (layer "F.Cu") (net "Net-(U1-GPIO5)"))
 (segment (start 67.19 67.335) (end 71.025 63.5) (width 0.2) (layer "F.Cu") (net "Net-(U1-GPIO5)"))
 (segment (start 113.25 85.25) (end 107.5 91) (width 0.2) (layer "F.Cu") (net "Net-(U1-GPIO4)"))
 (segment (start 113.25 70.5) (end 113.25 85.25) (width 0.2) (layer "F.Cu") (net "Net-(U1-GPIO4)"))
 (segment (start 107.5 91) (end 106.1 91) (width 0.2) (layer "F.Cu") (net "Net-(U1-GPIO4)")))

